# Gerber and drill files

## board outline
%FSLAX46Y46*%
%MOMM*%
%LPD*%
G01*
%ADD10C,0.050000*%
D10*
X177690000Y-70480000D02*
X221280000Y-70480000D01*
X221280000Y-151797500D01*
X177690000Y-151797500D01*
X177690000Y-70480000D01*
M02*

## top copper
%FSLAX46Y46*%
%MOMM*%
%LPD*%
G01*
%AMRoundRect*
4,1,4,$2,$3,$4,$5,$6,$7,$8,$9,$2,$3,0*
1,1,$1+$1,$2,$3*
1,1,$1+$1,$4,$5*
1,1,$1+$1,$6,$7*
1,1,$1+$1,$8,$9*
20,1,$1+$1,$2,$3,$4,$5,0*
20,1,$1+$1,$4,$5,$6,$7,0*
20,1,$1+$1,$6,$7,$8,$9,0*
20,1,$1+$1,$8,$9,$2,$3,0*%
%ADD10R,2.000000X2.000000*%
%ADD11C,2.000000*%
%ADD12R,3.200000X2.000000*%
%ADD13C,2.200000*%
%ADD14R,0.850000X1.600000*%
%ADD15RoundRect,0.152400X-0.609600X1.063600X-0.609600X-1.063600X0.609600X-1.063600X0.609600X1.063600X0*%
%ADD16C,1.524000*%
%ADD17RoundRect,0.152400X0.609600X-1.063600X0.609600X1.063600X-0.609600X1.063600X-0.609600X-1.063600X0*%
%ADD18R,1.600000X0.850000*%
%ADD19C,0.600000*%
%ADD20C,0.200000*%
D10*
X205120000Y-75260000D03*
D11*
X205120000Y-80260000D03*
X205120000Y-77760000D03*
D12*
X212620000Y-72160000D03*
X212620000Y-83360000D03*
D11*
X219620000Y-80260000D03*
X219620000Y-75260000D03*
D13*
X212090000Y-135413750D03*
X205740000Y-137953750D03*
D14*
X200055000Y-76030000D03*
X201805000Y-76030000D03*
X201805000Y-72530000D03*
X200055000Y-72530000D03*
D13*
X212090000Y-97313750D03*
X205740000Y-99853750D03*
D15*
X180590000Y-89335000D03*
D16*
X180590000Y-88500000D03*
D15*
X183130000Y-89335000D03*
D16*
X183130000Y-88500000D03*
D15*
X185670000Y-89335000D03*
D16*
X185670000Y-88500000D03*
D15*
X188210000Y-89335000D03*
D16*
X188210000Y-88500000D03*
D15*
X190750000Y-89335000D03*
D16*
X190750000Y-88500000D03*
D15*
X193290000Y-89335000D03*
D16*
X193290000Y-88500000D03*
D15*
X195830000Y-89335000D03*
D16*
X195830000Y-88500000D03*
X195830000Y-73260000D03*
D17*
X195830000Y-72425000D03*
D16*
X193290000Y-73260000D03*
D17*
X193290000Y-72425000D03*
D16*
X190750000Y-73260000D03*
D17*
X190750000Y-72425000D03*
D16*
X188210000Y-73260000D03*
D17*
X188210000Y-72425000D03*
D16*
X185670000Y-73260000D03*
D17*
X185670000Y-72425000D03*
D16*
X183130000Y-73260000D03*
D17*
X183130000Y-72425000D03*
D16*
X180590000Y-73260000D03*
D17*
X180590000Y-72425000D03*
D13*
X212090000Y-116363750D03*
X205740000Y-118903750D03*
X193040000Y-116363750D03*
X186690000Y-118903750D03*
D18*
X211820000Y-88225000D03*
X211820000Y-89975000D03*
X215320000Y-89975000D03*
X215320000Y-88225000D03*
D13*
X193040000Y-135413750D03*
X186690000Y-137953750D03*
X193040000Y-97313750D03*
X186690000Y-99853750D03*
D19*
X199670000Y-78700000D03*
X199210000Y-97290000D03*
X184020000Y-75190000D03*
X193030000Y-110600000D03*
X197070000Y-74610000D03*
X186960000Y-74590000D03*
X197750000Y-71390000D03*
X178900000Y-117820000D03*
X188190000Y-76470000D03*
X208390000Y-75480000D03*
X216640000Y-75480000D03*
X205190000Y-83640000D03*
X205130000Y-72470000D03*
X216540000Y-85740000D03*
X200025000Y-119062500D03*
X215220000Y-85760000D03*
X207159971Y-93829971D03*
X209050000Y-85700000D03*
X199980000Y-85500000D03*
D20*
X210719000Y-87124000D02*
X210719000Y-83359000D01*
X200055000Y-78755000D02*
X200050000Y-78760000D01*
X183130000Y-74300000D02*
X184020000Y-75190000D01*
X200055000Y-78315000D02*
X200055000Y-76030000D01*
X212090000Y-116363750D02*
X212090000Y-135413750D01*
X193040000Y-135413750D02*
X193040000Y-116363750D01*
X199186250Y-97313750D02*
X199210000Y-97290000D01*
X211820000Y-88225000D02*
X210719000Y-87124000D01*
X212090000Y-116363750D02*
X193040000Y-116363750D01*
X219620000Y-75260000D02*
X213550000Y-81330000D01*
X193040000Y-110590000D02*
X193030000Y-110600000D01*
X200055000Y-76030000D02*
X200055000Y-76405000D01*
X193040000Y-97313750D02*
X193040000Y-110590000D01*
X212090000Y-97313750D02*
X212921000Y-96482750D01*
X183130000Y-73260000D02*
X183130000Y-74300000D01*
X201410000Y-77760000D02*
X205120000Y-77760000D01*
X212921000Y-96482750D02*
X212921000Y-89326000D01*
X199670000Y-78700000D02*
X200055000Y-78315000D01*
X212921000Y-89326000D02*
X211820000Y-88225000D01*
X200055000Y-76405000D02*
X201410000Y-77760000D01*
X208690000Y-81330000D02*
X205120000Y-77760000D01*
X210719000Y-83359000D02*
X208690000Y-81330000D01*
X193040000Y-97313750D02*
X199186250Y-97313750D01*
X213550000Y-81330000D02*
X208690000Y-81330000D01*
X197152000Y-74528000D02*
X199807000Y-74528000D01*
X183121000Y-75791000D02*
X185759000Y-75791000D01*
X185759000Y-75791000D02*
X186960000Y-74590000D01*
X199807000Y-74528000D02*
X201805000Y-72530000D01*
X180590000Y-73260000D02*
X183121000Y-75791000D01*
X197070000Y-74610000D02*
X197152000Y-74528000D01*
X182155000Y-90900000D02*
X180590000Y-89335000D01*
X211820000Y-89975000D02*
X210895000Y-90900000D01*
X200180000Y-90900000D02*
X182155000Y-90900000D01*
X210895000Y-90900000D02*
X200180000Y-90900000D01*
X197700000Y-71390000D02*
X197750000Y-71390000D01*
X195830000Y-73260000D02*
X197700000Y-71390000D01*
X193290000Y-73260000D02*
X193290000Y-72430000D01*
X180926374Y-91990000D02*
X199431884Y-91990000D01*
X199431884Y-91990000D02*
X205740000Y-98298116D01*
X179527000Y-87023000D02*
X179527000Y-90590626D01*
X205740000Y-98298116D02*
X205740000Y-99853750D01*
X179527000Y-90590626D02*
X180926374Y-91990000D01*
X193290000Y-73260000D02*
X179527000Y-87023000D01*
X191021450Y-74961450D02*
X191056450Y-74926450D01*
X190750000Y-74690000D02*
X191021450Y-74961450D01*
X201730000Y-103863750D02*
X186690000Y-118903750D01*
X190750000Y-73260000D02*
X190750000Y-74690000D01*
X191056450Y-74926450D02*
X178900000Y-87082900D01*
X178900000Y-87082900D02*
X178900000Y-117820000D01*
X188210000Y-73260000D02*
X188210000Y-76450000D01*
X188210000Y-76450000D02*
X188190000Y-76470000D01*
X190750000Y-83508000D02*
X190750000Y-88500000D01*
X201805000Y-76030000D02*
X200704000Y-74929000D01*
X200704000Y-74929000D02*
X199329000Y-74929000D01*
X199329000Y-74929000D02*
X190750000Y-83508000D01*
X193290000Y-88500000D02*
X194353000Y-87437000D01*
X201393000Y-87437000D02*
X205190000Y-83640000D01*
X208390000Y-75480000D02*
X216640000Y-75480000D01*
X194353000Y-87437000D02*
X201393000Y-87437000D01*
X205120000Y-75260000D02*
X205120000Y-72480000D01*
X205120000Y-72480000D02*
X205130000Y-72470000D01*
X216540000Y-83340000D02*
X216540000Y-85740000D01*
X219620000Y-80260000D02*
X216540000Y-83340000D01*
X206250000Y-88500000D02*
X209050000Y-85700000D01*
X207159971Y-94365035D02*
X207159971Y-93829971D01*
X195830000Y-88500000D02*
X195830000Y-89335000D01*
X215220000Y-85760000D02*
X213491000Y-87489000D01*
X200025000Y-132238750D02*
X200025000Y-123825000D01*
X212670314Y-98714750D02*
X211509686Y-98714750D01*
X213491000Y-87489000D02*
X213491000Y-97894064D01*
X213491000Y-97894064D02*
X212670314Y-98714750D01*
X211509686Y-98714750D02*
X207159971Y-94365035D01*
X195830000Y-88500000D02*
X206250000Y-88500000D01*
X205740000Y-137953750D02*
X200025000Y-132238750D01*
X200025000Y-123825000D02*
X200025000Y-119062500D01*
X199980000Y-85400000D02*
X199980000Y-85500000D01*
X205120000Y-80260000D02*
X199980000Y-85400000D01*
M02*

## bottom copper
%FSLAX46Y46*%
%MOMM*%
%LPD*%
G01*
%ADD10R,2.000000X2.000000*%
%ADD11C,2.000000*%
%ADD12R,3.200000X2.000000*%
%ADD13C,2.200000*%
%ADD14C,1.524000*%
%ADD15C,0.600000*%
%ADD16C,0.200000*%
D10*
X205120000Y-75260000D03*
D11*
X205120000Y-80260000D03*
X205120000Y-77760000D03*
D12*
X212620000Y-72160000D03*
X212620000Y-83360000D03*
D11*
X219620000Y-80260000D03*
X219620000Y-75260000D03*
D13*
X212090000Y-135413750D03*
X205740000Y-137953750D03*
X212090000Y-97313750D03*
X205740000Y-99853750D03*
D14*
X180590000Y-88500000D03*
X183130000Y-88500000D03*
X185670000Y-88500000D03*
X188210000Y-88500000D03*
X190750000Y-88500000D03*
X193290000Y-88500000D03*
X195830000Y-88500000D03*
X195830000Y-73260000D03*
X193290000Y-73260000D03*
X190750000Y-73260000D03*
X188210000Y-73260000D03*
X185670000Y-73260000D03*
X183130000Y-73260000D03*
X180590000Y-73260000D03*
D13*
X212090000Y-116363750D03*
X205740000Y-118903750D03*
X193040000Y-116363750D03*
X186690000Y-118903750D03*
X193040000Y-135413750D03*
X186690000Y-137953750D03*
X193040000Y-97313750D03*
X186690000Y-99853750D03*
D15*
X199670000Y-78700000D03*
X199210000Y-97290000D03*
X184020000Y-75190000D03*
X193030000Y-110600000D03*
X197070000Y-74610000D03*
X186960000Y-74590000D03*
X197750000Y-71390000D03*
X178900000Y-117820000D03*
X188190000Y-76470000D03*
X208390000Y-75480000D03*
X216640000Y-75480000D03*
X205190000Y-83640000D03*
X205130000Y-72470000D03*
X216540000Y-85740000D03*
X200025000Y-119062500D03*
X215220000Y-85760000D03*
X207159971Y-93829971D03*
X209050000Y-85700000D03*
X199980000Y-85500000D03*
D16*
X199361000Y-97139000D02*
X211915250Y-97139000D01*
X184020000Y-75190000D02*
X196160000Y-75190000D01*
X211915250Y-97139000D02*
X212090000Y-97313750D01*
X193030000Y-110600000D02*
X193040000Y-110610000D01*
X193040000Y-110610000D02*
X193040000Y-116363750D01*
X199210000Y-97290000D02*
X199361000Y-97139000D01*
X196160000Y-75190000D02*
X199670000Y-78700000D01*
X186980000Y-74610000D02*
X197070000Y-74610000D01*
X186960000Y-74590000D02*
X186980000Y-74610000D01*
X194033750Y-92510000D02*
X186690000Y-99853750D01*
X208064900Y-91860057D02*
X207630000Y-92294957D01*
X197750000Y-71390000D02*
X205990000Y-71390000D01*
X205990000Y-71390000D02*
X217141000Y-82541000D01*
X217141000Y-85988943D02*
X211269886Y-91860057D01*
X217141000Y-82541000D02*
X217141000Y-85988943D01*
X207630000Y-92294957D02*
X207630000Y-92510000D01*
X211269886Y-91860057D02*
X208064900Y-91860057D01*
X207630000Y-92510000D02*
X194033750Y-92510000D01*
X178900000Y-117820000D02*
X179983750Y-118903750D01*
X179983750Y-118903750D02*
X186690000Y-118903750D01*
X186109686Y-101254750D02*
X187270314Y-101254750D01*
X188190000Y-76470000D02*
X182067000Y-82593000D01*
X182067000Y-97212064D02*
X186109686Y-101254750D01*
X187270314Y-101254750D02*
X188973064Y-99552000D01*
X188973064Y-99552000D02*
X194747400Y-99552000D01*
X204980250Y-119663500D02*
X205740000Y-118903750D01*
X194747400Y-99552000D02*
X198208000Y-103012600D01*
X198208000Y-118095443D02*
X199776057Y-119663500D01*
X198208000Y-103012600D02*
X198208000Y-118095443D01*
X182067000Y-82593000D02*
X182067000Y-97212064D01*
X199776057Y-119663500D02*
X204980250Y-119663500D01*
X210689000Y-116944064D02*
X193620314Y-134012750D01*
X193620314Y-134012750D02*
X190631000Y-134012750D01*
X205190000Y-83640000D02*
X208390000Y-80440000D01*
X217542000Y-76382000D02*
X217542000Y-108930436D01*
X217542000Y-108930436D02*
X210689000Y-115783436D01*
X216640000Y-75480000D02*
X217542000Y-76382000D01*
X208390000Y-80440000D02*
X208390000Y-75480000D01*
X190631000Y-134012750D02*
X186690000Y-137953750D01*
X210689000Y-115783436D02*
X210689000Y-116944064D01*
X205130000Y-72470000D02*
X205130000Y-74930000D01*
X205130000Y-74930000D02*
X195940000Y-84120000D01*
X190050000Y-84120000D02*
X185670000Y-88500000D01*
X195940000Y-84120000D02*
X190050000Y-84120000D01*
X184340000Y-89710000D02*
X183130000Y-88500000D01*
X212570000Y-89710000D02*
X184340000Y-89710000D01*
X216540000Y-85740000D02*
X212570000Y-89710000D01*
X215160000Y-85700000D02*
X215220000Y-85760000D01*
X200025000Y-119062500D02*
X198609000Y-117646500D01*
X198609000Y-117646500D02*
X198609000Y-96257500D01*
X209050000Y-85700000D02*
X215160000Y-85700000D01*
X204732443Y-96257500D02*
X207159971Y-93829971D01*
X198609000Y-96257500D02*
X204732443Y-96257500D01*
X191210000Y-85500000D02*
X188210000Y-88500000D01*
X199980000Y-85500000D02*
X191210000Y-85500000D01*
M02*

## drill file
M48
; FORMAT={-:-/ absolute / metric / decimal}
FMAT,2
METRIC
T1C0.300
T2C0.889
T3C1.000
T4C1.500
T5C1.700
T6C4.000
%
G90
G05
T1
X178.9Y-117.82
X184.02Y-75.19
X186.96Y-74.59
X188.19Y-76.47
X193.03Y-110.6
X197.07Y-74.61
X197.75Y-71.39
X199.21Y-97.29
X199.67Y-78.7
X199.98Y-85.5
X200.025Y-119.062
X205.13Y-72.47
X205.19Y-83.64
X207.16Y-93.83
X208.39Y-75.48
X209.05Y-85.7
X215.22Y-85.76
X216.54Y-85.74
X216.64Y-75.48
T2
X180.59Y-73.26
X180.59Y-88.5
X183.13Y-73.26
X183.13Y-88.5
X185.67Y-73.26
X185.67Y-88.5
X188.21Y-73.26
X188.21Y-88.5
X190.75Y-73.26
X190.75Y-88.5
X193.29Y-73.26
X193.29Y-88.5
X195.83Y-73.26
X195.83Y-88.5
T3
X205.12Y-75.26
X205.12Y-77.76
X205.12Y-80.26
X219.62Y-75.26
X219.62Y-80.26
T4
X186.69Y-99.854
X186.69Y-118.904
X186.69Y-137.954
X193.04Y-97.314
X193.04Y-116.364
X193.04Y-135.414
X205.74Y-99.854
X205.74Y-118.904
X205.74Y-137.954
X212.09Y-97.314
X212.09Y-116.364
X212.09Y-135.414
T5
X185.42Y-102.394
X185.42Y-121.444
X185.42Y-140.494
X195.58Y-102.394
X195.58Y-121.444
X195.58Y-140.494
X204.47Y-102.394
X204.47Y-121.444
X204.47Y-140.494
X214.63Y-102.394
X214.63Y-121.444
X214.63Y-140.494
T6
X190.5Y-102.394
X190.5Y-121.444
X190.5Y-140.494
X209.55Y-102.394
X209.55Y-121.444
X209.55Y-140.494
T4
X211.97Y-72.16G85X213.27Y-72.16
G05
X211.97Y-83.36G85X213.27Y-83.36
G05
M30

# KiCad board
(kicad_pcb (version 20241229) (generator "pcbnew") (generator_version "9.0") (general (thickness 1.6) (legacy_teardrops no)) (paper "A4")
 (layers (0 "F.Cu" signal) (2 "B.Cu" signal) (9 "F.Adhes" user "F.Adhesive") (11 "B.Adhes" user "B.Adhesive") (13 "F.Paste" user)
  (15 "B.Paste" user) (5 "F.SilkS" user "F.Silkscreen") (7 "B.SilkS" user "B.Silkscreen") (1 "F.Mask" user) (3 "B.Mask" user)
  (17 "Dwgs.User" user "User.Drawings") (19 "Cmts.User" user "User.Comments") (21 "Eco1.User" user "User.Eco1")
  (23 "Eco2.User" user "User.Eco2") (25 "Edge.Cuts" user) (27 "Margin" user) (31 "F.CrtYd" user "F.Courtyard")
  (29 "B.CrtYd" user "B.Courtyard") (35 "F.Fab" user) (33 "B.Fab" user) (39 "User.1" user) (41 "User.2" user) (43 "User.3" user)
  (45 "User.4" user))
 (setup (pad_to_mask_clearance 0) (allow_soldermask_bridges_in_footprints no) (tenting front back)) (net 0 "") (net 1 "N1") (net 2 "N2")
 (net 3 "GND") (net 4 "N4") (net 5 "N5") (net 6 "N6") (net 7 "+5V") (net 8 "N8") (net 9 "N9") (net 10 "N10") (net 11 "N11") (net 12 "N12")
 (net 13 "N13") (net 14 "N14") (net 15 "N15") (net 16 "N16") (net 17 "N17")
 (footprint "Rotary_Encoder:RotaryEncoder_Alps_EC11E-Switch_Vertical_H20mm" (layer "F.Cu") (at 205.12 75.26)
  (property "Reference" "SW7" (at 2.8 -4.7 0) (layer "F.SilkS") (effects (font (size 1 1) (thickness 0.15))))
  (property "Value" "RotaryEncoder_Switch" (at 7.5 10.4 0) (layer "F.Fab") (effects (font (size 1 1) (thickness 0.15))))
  (pad "A" thru_hole rect (at 0 0) (size 2 2) (drill 1) (layers "*.Cu" "*.Mask") (remove_unused_layers no) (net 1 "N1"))
  (pad "B" thru_hole circle (at 0 5) (size 2 2) (drill 1) (layers "*.Cu" "*.Mask") (remove_unused_layers no) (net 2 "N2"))
  (pad "C" thru_hole circle (at 0 2.5) (size 2 2) (drill 1) (layers "*.Cu" "*.Mask") (remove_unused_layers no) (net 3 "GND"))
  (pad "MP" thru_hole rect (at 7.5 -3.1) (size 3.2 2) (drill oval 2.8 1.5) (layers "*.Cu" "*.Mask") (remove_unused_layers no))
  (pad "MP" thru_hole rect (at 7.5 8.1) (size 3.2 2) (drill oval 2.8 1.5) (layers "*.Cu" "*.Mask") (remove_unused_layers no))
  (pad "S1" thru_hole circle (at 14.5 5) (size 2 2) (drill 1) (layers "*.Cu" "*.Mask") (remove_unused_layers no) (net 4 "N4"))
  (pad "S2" thru_hole circle (at 14.5 0) (size 2 2) (drill 1) (layers "*.Cu" "*.Mask") (remove_unused_layers no) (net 3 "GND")))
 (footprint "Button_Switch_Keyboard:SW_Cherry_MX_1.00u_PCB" (layer "F.Cu") (at 212.09 135.41375)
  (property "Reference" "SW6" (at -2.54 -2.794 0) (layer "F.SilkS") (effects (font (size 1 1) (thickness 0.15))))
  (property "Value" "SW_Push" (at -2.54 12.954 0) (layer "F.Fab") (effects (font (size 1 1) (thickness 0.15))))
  (pad "" np_thru_hole circle (at -7.62 5.08) (size 1.7 1.7) (drill 1.7) (layers "*.Cu" "*.Mask"))
  (pad "" np_thru_hole circle (at -2.54 5.08) (size 4 4) (drill 4) (layers "*.Cu" "*.Mask"))
  (pad "" np_thru_hole circle (at 2.54 5.08) (size 1.7 1.7) (drill 1.7) (layers "*.Cu" "*.Mask"))
  (pad "1" thru_hole circle (at 0 0) (size 2.2 2.2) (drill 1.5) (layers "*.Cu" "*.Mask") (remove_unused_layers no) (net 3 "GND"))
  (pad "2" thru_hole circle (at -6.35 2.54) (size 2.2 2.2) (drill 1.5) (layers "*.Cu" "*.Mask") (remove_unused_layers no) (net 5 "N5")))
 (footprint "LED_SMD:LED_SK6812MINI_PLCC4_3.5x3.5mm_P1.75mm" (layer "F.Cu") (at 200.93 74.28 90)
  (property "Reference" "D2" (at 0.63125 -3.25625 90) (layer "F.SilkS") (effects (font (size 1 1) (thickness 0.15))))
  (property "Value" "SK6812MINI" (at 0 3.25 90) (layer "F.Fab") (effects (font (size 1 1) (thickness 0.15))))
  (pad "1" smd rect (at -1.75 -0.875 90) (size 1.6 0.85) (layers "F.Cu" "F.Mask" "F.Paste") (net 3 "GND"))
  (pad "2" smd rect (at -1.75 0.875 90) (size 1.6 0.85) (layers "F.Cu" "F.Mask" "F.Paste") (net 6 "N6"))
  (pad "3" smd rect (at 1.75 0.875 90) (size 1.6 0.85) (layers "F.Cu" "F.Mask" "F.Paste") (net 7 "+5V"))
  (pad "4" smd rect (at 1.75 -0.875 90) (size 1.6 0.85) (layers "F.Cu" "F.Mask" "F.Paste") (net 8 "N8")))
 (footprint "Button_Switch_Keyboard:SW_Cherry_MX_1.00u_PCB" (layer "F.Cu") (at 212.09 97.31375)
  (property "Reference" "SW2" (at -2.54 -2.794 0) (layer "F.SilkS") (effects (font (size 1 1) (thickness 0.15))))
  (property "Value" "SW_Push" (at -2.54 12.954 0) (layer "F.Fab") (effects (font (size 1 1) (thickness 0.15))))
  (pad "" np_thru_hole circle (at -7.62 5.08) (size 1.7 1.7) (drill 1.7) (layers "*.Cu" "*.Mask"))
  (pad "" np_thru_hole circle (at -2.54 5.08) (size 4 4) (drill 4) (layers "*.Cu" "*.Mask"))
  (pad "" np_thru_hole circle (at 2.54 5.08) (size 1.7 1.7) (drill 1.7) (layers "*.Cu" "*.Mask"))
  (pad "1" thru_hole circle (at 0 0) (size 2.2 2.2) (drill 1.5) (layers "*.Cu" "*.Mask") (remove_unused_layers no) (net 3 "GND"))
  (pad "2" thru_hole circle (at -6.35 2.54) (size 2.2 2.2) (drill 1.5) (layers "*.Cu" "*.Mask") (remove_unused_layers no) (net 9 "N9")))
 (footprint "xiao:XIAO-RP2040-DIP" (layer "F.Cu") (at 188.21 80.88 90)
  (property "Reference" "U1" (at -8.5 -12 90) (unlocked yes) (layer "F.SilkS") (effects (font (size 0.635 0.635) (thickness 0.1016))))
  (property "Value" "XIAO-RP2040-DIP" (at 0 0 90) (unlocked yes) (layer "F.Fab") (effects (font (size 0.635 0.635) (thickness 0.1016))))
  (pad "1" smd roundrect (at -8.455 -7.62 270) (size 2.432 1.524) (layers "F.Cu" "F.Mask") (roundrect_rratio 0.1) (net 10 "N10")
   (thermal_bridge_angle 45))
  (pad "1" thru_hole circle (at -7.62 -7.62 270) (size 1.524 1.524) (drill 0.889) (layers "*.Cu" "*.Mask") (remove_unused_layers no)
   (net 10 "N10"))
  (pad "2" smd roundrect (at -8.455 -5.08 270) (size 2.432 1.524) (layers "F.Cu" "F.Mask") (roundrect_rratio 0.1) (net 4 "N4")
   (thermal_bridge_angle 45))
  (pad "2" thru_hole circle (at -7.62 -5.08 270) (size 1.524 1.524) (drill 0.889) (layers "*.Cu" "*.Mask") (remove_unused_layers no)
   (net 4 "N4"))
  (pad "3" smd roundrect (at -8.455 -2.54 270) (size 2.432 1.524) (layers "F.Cu" "F.Mask") (roundrect_rratio 0.1) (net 1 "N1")
   (thermal_bridge_angle 45))
  (pad "3" thru_hole circle (at -7.62 -2.54 270) (size 1.524 1.524) (drill 0.889) (layers "*.Cu" "*.Mask") (remove_unused_layers no)
   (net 1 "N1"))
  (pad "4" smd roundrect (at -8.455 0 270) (size 2.432 1.524) (layers "F.Cu" "F.Mask") (roundrect_rratio 0.1) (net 2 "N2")
   (thermal_bridge_angle 45))
  (pad "4" thru_hole circle (at -7.62 0 270) (size 1.524 1.524) (drill 0.889) (layers "*.Cu" "*.Mask") (remove_unused_layers no)
   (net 2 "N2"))
  (pad "5" smd roundrect (at -8.455 2.54 270) (size 2.432 1.524) (layers "F.Cu" "F.Mask") (roundrect_rratio 0.1) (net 6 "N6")
   (thermal_bridge_angle 45))
  (pad "5" thru_hole circle (at -7.62 2.54 270) (size 1.524 1.524) (drill 0.889) (layers "*.Cu" "*.Mask") (remove_unused_layers no)
   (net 6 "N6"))
  (pad "6" smd roundrect (at -8.455 5.08 270) (size 2.432 1.524) (layers "F.Cu" "F.Mask") (roundrect_rratio 0.1) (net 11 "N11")
   (thermal_bridge_angle 45))
  (pad "6" thru_hole circle (at -7.62 5.08 270) (size 1.524 1.524) (drill 0.889) (layers "*.Cu" "*.Mask") (remove_unused_layers no)
   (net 11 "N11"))
  (pad "7" smd roundrect (at -8.455 7.62 270) (size 2.432 1.524) (layers "F.Cu" "F.Mask") (roundrect_rratio 0.1) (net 5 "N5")
   (thermal_bridge_angle 45))
  (pad "7" thru_hole circle (at -7.62 7.62 270) (size 1.524 1.524) (drill 0.889) (layers "*.Cu" "*.Mask") (remove_unused_layers no)
   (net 5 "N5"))
  (pad "8" thru_hole circle (at 7.62 7.62 90) (size 1.524 1.524) (drill 0.889) (layers "*.Cu" "*.Mask") (remove_unused_layers no)
   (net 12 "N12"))
  (pad "8" smd roundrect (at 8.455 7.62 90) (size 2.432 1.524) (layers "F.Cu" "F.Mask") (roundrect_rratio 0.1) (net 12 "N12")
   (thermal_bridge_angle 45))
  (pad "9" thru_hole circle (at 7.62 5.08 90) (size 1.524 1.524) (drill 0.889) (layers "*.Cu" "*.Mask") (remove_unused_layers no)
   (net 9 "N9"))
  (pad "9" smd roundrect (at 8.455 5.08 90) (size 2.432 1.524) (layers "F.Cu" "F.Mask") (roundrect_rratio 0.1) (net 9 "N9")
   (thermal_bridge_angle 45))
  (pad "10" thru_hole circle (at 7.62 2.54 90) (size 1.524 1.524) (drill 0.889) (layers "*.Cu" "*.Mask") (remove_unused_layers no)
   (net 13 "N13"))
  (pad "10" smd roundrect (at 8.455 2.54 90) (size 2.432 1.524) (layers "F.Cu" "F.Mask") (roundrect_rratio 0.1) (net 13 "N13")
   (thermal_bridge_angle 45))
  (pad "11" thru_hole circle (at 7.62 0 90) (size 1.524 1.524) (drill 0.889) (layers "*.Cu" "*.Mask") (remove_unused_layers no)
   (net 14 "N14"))
  (pad "11" smd roundrect (at 8.455 0 90) (size 2.432 1.524) (layers "F.Cu" "F.Mask") (roundrect_rratio 0.1) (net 14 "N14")
   (thermal_bridge_angle 45))
  (pad "12" thru_hole circle (at 7.62 -2.54 90) (size 1.524 1.524) (drill 0.889) (layers "*.Cu" "*.Mask") (remove_unused_layers no)
   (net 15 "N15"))
  (pad "12" smd roundrect (at 8.455 -2.54 90) (size 2.432 1.524) (layers "F.Cu" "F.Mask") (roundrect_rratio 0.1) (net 15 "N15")
   (thermal_bridge_angle 45))
  (pad "13" thru_hole circle (at 7.62 -5.08 90) (size 1.524 1.524) (drill 0.889) (layers "*.Cu" "*.Mask") (remove_unused_layers no)
   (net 3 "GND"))
  (pad "13" smd roundrect (at 8.455 -5.08 90) (size 2.432 1.524) (layers "F.Cu" "F.Mask") (roundrect_rratio 0.1) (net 3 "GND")
   (thermal_bridge_angle 45))
  (pad "14" thru_hole circle (at 7.62 -7.62 90) (size 1.524 1.524) (drill 0.889) (layers "*.Cu" "*.Mask") (remove_unused_layers no)
   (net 7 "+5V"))
  (pad "14" smd roundrect (at 8.455 -7.62 90) (size 2.432 1.524) (layers "F.Cu" "F.Mask") (roundrect_rratio 0.1) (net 7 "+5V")
   (thermal_bridge_angle 45)))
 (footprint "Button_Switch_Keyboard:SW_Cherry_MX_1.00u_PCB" (layer "F.Cu") (at 212.09 116.36375)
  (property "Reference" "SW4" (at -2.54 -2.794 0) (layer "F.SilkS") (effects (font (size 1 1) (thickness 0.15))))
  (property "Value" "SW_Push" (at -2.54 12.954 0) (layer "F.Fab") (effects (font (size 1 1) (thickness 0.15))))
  (pad "" np_thru_hole circle (at -7.62 5.08) (size 1.7 1.7) (drill 1.7) (layers "*.Cu" "*.Mask"))
  (pad "" np_thru_hole circle (at -2.54 5.08) (size 4 4) (drill 4) (layers "*.Cu" "*.Mask"))
  (pad "" np_thru_hole circle (at 2.54 5.08) (size 1.7 1.7) (drill 1.7) (layers "*.Cu" "*.Mask"))
  (pad "1" thru_hole circle (at 0 0) (size 2.2 2.2) (drill 1.5) (layers "*.Cu" "*.Mask") (remove_unused_layers no) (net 3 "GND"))
  (pad "2" thru_hole circle (at -6.35 2.54) (size 2.2 2.2) (drill 1.5) (layers "*.Cu" "*.Mask") (remove_unused_layers no) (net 14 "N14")))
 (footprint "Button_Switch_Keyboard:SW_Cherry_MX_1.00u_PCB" (layer "F.Cu") (at 193.04 116.36375)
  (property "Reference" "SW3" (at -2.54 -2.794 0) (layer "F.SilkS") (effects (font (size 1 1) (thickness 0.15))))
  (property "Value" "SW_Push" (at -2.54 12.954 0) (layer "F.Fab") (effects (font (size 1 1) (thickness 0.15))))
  (pad "" np_thru_hole circle (at -7.62 5.08) (size 1.7 1.7) (drill 1.7) (layers "*.Cu" "*.Mask"))
  (pad "" np_thru_hole circle (at -2.54 5.08) (size 4 4) (drill 4) (layers "*.Cu" "*.Mask"))
  (pad "" np_thru_hole circle (at 2.54 5.08) (size 1.7 1.7) (drill 1.7) (layers "*.Cu" "*.Mask"))
  (pad "1" thru_hole circle (at 0 0) (size 2.2 2.2) (drill 1.5) (layers "*.Cu" "*.Mask") (remove_unused_layers no) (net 3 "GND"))
  (pad "2" thru_hole circle (at -6.35 2.54) (size 2.2 2.2) (drill 1.5) (layers "*.Cu" "*.Mask") (remove_unused_layers no) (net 13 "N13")))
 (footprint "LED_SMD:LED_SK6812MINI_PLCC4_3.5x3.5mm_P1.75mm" (layer "F.Cu") (at 213.57 89.1)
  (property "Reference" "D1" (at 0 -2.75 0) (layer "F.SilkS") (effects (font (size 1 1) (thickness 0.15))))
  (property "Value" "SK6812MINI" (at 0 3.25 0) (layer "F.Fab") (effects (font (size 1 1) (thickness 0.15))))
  (pad "1" smd rect (at -1.75 -0.875) (size 1.6 0.85) (layers "F.Cu" "F.Mask" "F.Paste") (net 3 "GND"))
  (pad "2" smd rect (at -1.75 0.875) (size 1.6 0.85) (layers "F.Cu" "F.Mask" "F.Paste") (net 10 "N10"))
  (pad "3" smd rect (at 1.75 0.875) (size 1.6 0.85) (layers "F.Cu" "F.Mask" "F.Paste") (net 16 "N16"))
  (pad "4" smd rect (at 1.75 -0.875) (size 1.6 0.85) (layers "F.Cu" "F.Mask" "F.Paste") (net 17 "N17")))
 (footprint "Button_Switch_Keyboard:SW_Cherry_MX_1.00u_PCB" (layer "F.Cu") (at 193.04 135.41375)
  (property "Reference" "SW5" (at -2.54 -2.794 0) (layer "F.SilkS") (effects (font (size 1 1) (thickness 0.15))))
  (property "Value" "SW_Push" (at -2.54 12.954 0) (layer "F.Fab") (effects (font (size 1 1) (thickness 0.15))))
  (pad "" np_thru_hole circle (at -7.62 5.08) (size 1.7 1.7) (drill 1.7) (layers "*.Cu" "*.Mask"))
  (pad "" np_thru_hole circle (at -2.54 5.08) (size 4 4) (drill 4) (layers "*.Cu" "*.Mask"))
  (pad "" np_thru_hole circle (at 2.54 5.08) (size 1.7 1.7) (drill 1.7) (layers "*.Cu" "*.Mask"))
  (pad "1" thru_hole circle (at 0 0) (size 2.2 2.2) (drill 1.5) (layers "*.Cu" "*.Mask") (remove_unused_layers no) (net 3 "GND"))
  (pad "2" thru_hole circle (at -6.35 2.54) (size 2.2 2.2) (drill 1.5) (layers "*.Cu" "*.Mask") (remove_unused_layers no) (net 11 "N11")))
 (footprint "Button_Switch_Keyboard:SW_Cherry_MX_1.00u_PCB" (layer "F.Cu") (at 193.04 97.31375)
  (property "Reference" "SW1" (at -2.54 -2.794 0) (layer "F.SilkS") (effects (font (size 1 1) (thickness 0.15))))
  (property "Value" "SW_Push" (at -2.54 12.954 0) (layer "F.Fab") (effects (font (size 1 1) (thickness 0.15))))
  (pad "" np_thru_hole circle (at -7.62 5.08) (size 1.7 1.7) (drill 1.7) (layers "*.Cu" "*.Mask"))
  (pad "" np_thru_hole circle (at -2.54 5.08) (size 4 4) (drill 4) (layers "*.Cu" "*.Mask"))
  (pad "" np_thru_hole circle (at 2.54 5.08) (size 1.7 1.7) (drill 1.7) (layers "*.Cu" "*.Mask"))
  (pad "1" thru_hole circle (at 0 0) (size 2.2 2.2) (drill 1.5) (layers "*.Cu" "*.Mask") (remove_unused_layers no) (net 3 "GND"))
  (pad "2" thru_hole circle (at -6.35 2.54) (size 2.2 2.2) (drill 1.5) (layers "*.Cu" "*.Mask") (remove_unused_layers no) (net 12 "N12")))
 (gr_rect (start 177.69 70.48) (end 221.28 151.7975) (stroke (width 0.05) (type solid)) (fill no) (layer "Edge.Cuts"))
 (segment (start 210.719 87.124) (end 210.719 83.359) (width 0.2) (layer "F.Cu") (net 3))
 (segment (start 200.055 78.755) (end 200.05 78.76) (width 0.2) (layer "F.Cu") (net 3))
 (segment (start 183.13 74.3) (end 184.02 75.19) (width 0.2) (layer "F.Cu") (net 3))
 (segment (start 200.055 78.315) (end 200.055 76.03) (width 0.2) (layer "F.Cu") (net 3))
 (segment (start 212.09 116.36375) (end 212.09 135.41375) (width 0.2) (layer "F.Cu") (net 3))
 (segment (start 193.04 135.41375) (end 193.04 116.36375) (width 0.2) (layer "F.Cu") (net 3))
 (segment (start 199.18625 97.31375) (end 199.21 97.29) (width 0.2) (layer "F.Cu") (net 3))
 (segment (start 211.82 88.225) (end 210.719 87.124) (width 0.2) (layer "F.Cu") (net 3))
 (segment (start 212.09 116.36375) (end 193.04 116.36375) (width 0.2) (layer "F.Cu") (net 3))
 (segment (start 219.62 75.26) (end 213.55 81.33) (width 0.2) (layer "F.Cu") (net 3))
 (segment (start 193.04 110.59) (end 193.03 110.6) (width 0.2) (layer "F.Cu") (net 3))
 (segment (start 200.055 76.03) (end 200.055 76.405) (width 0.2) (layer "F.Cu") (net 3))
 (segment (start 193.04 97.31375) (end 193.04 110.59) (width 0.2) (layer "F.Cu") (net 3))
 (segment (start 212.09 97.31375) (end 212.921 96.48275) (width 0.2) (layer "F.Cu") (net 3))
 (segment (start 183.13 73.26) (end 183.13 74.3) (width 0.2) (layer "F.Cu") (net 3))
 (segment (start 201.41 77.76) (end 205.12 77.76) (width 0.2) (layer "F.Cu") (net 3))
 (segment (start 212.921 96.48275) (end 212.921 89.326) (width 0.2) (layer "F.Cu") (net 3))
 (segment (start 199.67 78.7) (end 200.055 78.315) (width 0.2) (layer "F.Cu") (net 3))
 (segment (start 212.921 89.326) (end 211.82 88.225) (width 0.2) (layer "F.Cu") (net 3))
 (segment (start 200.055 76.405) (end 201.41 77.76) (width 0.2) (layer "F.Cu") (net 3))
 (segment (start 208.69 81.33) (end 205.12 77.76) (width 0.2) (layer "F.Cu") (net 3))
 (segment (start 210.719 83.359) (end 208.69 81.33) (width 0.2) (layer "F.Cu") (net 3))
 (segment (start 193.04 97.31375) (end 199.18625 97.31375) (width 0.2) (layer "F.Cu") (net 3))
 (segment (start 213.55 81.33) (end 208.69 81.33) (width 0.2) (layer "F.Cu") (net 3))
 (via (at 199.67 78.7) (size 0.6) (drill 0.3) (layers "F.Cu" "B.Cu") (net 3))
 (via (at 199.21 97.29) (size 0.6) (drill 0.3) (layers "F.Cu" "B.Cu") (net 3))
 (via (at 184.02 75.19) (size 0.6) (drill 0.3) (layers "F.Cu" "B.Cu") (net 3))
 (via (at 193.03 110.6) (size 0.6) (drill 0.3) (layers "F.Cu" "B.Cu") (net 3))
 (segment (start 199.361 97.139) (end 211.91525 97.139) (width 0.2) (layer "B.Cu") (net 3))
 (segment (start 184.02 75.19) (end 196.16 75.19) (width 0.2) (layer "B.Cu") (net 3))
 (segment (start 211.91525 97.139) (end 212.09 97.31375) (width 0.2) (layer "B.Cu") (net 3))
 (segment (start 193.03 110.6) (end 193.04 110.61) (width 0.2) (layer "B.Cu") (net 3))
 (segment (start 193.04 110.61) (end 193.04 116.36375) (width 0.2) (layer "B.Cu") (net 3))
 (segment (start 199.21 97.29) (end 199.361 97.139) (width 0.2) (layer "B.Cu") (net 3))
 (segment (start 196.16 75.19) (end 199.67 78.7) (width 0.2) (layer "B.Cu") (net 3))
 (segment (start 197.152 74.528) (end 199.807 74.528) (width 0.2) (layer "F.Cu") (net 7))
 (segment (start 183.121 75.791) (end 185.759 75.791) (width 0.2) (layer "F.Cu") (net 7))
 (segment (start 185.759 75.791) (end 186.96 74.59) (width 0.2) (layer "F.Cu") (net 7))
 (segment (start 199.807 74.528) (end 201.805 72.53) (width 0.2) (layer "F.Cu") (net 7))
 (segment (start 180.59 73.26) (end 183.121 75.791) (width 0.2) (layer "F.Cu") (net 7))
 (segment (start 197.07 74.61) (end 197.152 74.528) (width 0.2) (layer "F.Cu") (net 7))
 (via (at 197.07 74.61) (size 0.6) (drill 0.3) (layers "F.Cu" "B.Cu") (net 7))
 (via (at 186.96 74.59) (size 0.6) (drill 0.3) (layers "F.Cu" "B.Cu") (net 7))
 (segment (start 186.98 74.61) (end 197.07 74.61) (width 0.2) (layer "B.Cu") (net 7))
 (segment (start 186.96 74.59) (end 186.98 74.61) (width 0.2) (layer "B.Cu") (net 7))
 (segment (start 182.155 90.9) (end 180.59 89.335) (width 0.2) (layer "F.Cu") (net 10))
 (segment (start 211.82 89.975) (end 210.895 90.9) (width 0.2) (layer "F.Cu") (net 10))
 (segment (start 200.18 90.9) (end 182.155 90.9) (width 0.2) (layer "F.Cu") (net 10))
 (segment (start 210.895 90.9) (end 200.18 90.9) (width 0.2) (layer "F.Cu") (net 10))
 (segment (start 197.7 71.39) (end 197.75 71.39) (width 0.2) (layer "F.Cu") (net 12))
 (segment (start 195.83 73.26) (end 197.7 71.39) (width 0.2) (layer "F.Cu") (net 12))
 (via (at 197.75 71.39) (size 0.6) (drill 0.3) (layers "F.Cu" "B.Cu") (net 12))
 (segment (start 194.03375 92.51) (end 186.69 99.85375) (width 0.2) (layer "B.Cu") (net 12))
 (segment (start 208.0649 91.860057) (end 207.63 92.294957) (width 0.2) (layer "B.Cu") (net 12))
 (segment (start 197.75 71.39) (end 205.99 71.39) (width 0.2) (layer "B.Cu") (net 12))
 (segment (start 205.99 71.39) (end 217.141 82.541) (width 0.2) (layer "B.Cu") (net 12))
 (segment (start 217.141 85.988943) (end 211.269886 91.860057) (width 0.2) (layer "B.Cu") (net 12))
 (segment (start 217.141 82.541) (end 217.141 85.988943) (width 0.2) (layer "B.Cu") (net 12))
 (segment (start 207.63 92.294957) (end 207.63 92.51) (width 0.2) (layer "B.Cu") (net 12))
 (segment (start 211.269886 91.860057) (end 208.0649 91.860057) (width 0.2) (layer "B.Cu") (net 12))
 (segment (start 207.63 92.51) (end 194.03375 92.51) (width 0.2) (layer "B.Cu") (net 12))
 (segment (start 193.29 73.26) (end 193.29 72.43) (width 0.2) (layer "F.Cu") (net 9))
 (segment (start 180.926374 91.99) (end 199.431884 91.99) (width 0.2) (layer "F.Cu") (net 9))
 (segment (start 199.431884 91.99) (end 205.74 98.298116) (width 0.2) (layer "F.Cu") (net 9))
 (segment (start 179.527 87.023) (end 179.527 90.590626) (width 0.2) (layer "F.Cu") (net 9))
 (segment (start 205.74 98.298116) (end 205.74 99.85375) (width 0.2) (layer "F.Cu") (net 9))
 (segment (start 179.527 90.590626) (end 180.926374 91.99) (width 0.2) (layer "F.Cu") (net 9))
 (segment (start 193.29 73.26) (end 179.527 87.023) (width 0.2) (layer "F.Cu") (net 9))
 (segment (start 191.02145 74.96145) (end 191.05645 74.92645) (width 0.2) (layer "F.Cu") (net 13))
 (segment (start 190.75 74.69) (end 191.02145 74.96145) (width 0.2) (layer "F.Cu") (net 13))
 (segment (start 201.73 103.86375) (end 186.69 118.90375) (width 0.2) (layer "F.Cu") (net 13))
 (segment (start 190.75 73.26) (end 190.75 74.69) (width 0.2) (layer "F.Cu") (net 13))
 (segment (start 191.05645 74.92645) (end 178.9 87.0829) (width 0.2) (layer "F.Cu") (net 13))
 (segment (start 178.9 87.0829) (end 178.9 117.82) (width 0.2) (layer "F.Cu") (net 13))
 (via (at 178.9 117.82) (size 0.6) (drill 0.3) (layers "F.Cu" "B.Cu") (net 13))
 (segment (start 178.9 117.82) (end 179.98375 118.90375) (width 0.2) (layer "B.Cu") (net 13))
 (segment (start 179.98375 118.90375) (end 186.69 118.90375) (width 0.2) (layer "B.Cu") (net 13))
 (segment (start 188.21 73.26) (end 188.21 76.45) (width 0.2) (layer "F.Cu") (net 14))
 (segment (start 188.21 76.45) (end 188.19 76.47) (width 0.2) (layer "F.Cu") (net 14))
 (via (at 188.19 76.47) (size 0.6) (drill 0.3) (layers "F.Cu" "B.Cu") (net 14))
 (segment (start 186.109686 101.25475) (end 187.270314 101.25475) (width 0.2) (layer "B.Cu") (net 14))
 (segment (start 188.19 76.47) (end 182.067 82.593) (width 0.2) (layer "B.Cu") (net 14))
 (segment (start 182.067 97.212064) (end 186.109686 101.25475) (width 0.2) (layer "B.Cu") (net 14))
 (segment (start 187.270314 101.25475) (end 188.973064 99.552) (width 0.2) (layer "B.Cu") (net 14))
 (segment (start 188.973064 99.552) (end 194.7474 99.552) (width 0.2) (layer "B.Cu") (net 14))
 (segment (start 204.98025 119.6635) (end 205.74 118.90375) (width 0.2) (layer "B.Cu") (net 14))
 (segment (start 194.7474 99.552) (end 198.208 103.0126) (width 0.2) (layer "B.Cu") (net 14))
 (segment (start 198.208 118.095443) (end 199.776057 119.6635) (width 0.2) (layer "B.Cu") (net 14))
 (segment (start 198.208 103.0126) (end 198.208 118.095443) (width 0.2) (layer "B.Cu") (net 14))
 (segment (start 182.067 82.593) (end 182.067 97.212064) (width 0.2) (layer "B.Cu") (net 14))
 (segment (start 199.776057 119.6635) (end 204.98025 119.6635) (width 0.2) (layer "B.Cu") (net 14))
 (segment (start 190.75 83.508) (end 190.75 88.5) (width 0.2) (layer "F.Cu") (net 6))
 (segment (start 201.805 76.03) (end 200.704 74.929) (width 0.2) (layer "F.Cu") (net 6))
 (segment (start 200.704 74.929) (end 199.329 74.929) (width 0.2) (layer "F.Cu") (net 6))
 (segment (start 199.329 74.929) (end 190.75 83.508) (width 0.2) (layer "F.Cu") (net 6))
 (segment (start 193.29 88.5) (end 194.353 87.437) (width 0.2) (layer "F.Cu") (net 11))
 (segment (start 201.393 87.437) (end 205.19 83.64) (width 0.2) (layer "F.Cu") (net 11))
 (segment (start 208.39 75.48) (end 216.64 75.48) (width 0.2) (layer "F.Cu") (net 11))
 (segment (start 194.353 87.437) (end 201.393 87.437) (width 0.2) (layer "F.Cu") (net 11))
 (via (at 208.39 75.48) (size 0.6) (drill 0.3) (layers "F.Cu" "B.Cu") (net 11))
 (via (at 216.64 75.48) (size 0.6) (drill 0.3) (layers "F.Cu" "B.Cu") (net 11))
 (via (at 205.19 83.64) (size 0.6) (drill 0.3) (layers "F.Cu" "B.Cu") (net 11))
 (segment (start 210.689 116.944064) (end 193.620314 134.01275) (width 0.2) (layer "B.Cu") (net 11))
 (segment (start 193.620314 134.01275) (end 190.631 134.01275) (width 0.2) (layer "B.Cu") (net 11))
 (segment (start 205.19 83.64) (end 208.39 80.44) (width 0.2) (layer "B.Cu") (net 11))
 (segment (start 217.542 76.382) (end 217.542 108.930436) (width 0.2) (layer "B.Cu") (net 11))
 (segment (start 217.542 108.930436) (end 210.689 115.783436) (width 0.2) (layer "B.Cu") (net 11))
 (segment (start 216.64 75.48) (end 217.542 76.382) (width 0.2) (layer "B.Cu") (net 11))
 (segment (start 208.39 80.44) (end 208.39 75.48) (width 0.2) (layer "B.Cu") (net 11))
 (segment (start 190.631 134.01275) (end 186.69 137.95375) (width 0.2) (layer "B.Cu") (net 11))
 (segment (start 210.689 115.783436) (end 210.689 116.944064) (width 0.2) (layer "B.Cu") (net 11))
 (segment (start 205.12 75.26) (end 205.12 72.48) (width 0.2) (layer "F.Cu") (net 1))
 (segment (start 205.12 72.48) (end 205.13 72.47) (width 0.2) (layer "F.Cu") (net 1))
 (via (at 205.13 72.47) (size 0.6) (drill 0.3) (layers "F.Cu" "B.Cu") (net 1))
 (segment (start 205.13 72.47) (end 205.13 74.93) (width 0.2) (layer "B.Cu") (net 1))
 (segment (start 205.13 74.93) (end 195.94 84.12) (width 0.2) (layer "B.Cu") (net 1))
 (segment (start 190.05 84.12) (end 185.67 88.5) (width 0.2) (layer "B.Cu") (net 1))
 (segment (start 195.94 84.12) (end 190.05 84.12) (width 0.2) (layer "B.Cu") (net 1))
 (segment (start 216.54 83.34) (end 216.54 85.74) (width 0.2) (layer "F.Cu") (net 4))
 (segment (start 219.62 80.26) (end 216.54 83.34) (width 0.2) (layer "F.Cu") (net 4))
 (via (at 216.54 85.74) (size 0.6) (drill 0.3) (layers "F.Cu" "B.Cu") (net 4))
 (segment (start 184.34 89.71) (end 183.13 88.5) (width 0.2) (layer "B.Cu") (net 4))
 (segment (start 212.57 89.71) (end 184.34 89.71) (width 0.2) (layer "B.Cu") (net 4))
 (segment (start 216.54 85.74) (end 212.57 89.71) (width 0.2) (layer "B.Cu") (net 4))
 (segment (start 206.25 88.5) (end 209.05 85.7) (width 0.2) (layer "F.Cu") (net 5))
 (segment (start 207.159971 94.365035) (end 207.159971 93.829971) (width 0.2) (layer "F.Cu") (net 5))
 (segment (start 195.83 88.5) (end 195.83 89.335) (width 0.2) (layer "F.Cu") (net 5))
 (segment (start 215.22 85.76) (end 213.491 87.489) (width 0.2) (layer "F.Cu") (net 5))
 (segment (start 200.025 132.23875) (end 200.025 123.825) (width 0.2) (layer "F.Cu") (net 5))
 (segment (start 212.670314 98.71475) (end 211.509686 98.71475) (width 0.2) (layer "F.Cu") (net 5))
 (segment (start 213.491 87.489) (end 213.491 97.894064) (width 0.2) (layer "F.Cu") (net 5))
 (segment (start 213.491 97.894064) (end 212.670314 98.71475) (width 0.2) (layer "F.Cu") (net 5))
 (segment (start 211.509686 98.71475) (end 207.159971 94.365035) (width 0.2) (layer "F.Cu") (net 5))
 (segment (start 195.83 88.5) (end 206.25 88.5) (width 0.2) (layer "F.Cu") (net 5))
 (segment (start 205.74 137.95375) (end 200.025 132.23875) (width 0.2) (layer "F.Cu") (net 5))
 (segment (start 200.025 123.825) (end 200.025 119.0625) (width 0.2) (layer "F.Cu") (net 5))
 (via (at 200.025 119.0625) (size 0.6) (drill 0.3) (layers "F.Cu" "B.Cu") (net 5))
 (via (at 215.22 85.76) (size 0.6) (drill 0.3) (layers "F.Cu" "B.Cu") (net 5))
 (via (at 207.159971 93.829971) (size 0.6) (drill 0.3) (layers "F.Cu" "B.Cu") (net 5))
 (via (at 209.05 85.7) (size 0.6) (drill 0.3) (layers "F.Cu" "B.Cu") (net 5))
 (segment (start 215.16 85.7) (end 215.22 85.76) (width 0.2) (layer "B.Cu") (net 5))
 (segment (start 200.025 119.0625) (end 198.609 117.6465) (width 0.2) (layer "B.Cu") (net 5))
 (segment (start 198.609 117.6465) (end 198.609 96.2575) (width 0.2) (layer "B.Cu") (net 5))
 (segment (start 209.05 85.7) (end 215.16 85.7) (width 0.2) (layer "B.Cu") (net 5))
 (segment (start 204.732443 96.2575) (end 207.159971 93.829971) (width 0.2) (layer "B.Cu") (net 5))
 (segment (start 198.609 96.2575) (end 204.732443 96.2575) (width 0.2) (layer "B.Cu") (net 5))
 (segment (start 199.98 85.4) (end 199.98 85.5) (width 0.2) (layer "F.Cu") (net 2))
 (segment (start 205.12 80.26) (end 199.98 85.4) (width 0.2) (layer "F.Cu") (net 2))
 (via (at 199.98 85.5) (size 0.6) (drill 0.3) (layers "F.Cu" "B.Cu") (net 2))
 (segment (start 191.21 85.5) (end 188.21 88.5) (width 0.2) (layer "B.Cu") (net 2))
 (segment (start 199.98 85.5) (end 191.21 85.5) (width 0.2) (layer "B.Cu") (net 2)))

